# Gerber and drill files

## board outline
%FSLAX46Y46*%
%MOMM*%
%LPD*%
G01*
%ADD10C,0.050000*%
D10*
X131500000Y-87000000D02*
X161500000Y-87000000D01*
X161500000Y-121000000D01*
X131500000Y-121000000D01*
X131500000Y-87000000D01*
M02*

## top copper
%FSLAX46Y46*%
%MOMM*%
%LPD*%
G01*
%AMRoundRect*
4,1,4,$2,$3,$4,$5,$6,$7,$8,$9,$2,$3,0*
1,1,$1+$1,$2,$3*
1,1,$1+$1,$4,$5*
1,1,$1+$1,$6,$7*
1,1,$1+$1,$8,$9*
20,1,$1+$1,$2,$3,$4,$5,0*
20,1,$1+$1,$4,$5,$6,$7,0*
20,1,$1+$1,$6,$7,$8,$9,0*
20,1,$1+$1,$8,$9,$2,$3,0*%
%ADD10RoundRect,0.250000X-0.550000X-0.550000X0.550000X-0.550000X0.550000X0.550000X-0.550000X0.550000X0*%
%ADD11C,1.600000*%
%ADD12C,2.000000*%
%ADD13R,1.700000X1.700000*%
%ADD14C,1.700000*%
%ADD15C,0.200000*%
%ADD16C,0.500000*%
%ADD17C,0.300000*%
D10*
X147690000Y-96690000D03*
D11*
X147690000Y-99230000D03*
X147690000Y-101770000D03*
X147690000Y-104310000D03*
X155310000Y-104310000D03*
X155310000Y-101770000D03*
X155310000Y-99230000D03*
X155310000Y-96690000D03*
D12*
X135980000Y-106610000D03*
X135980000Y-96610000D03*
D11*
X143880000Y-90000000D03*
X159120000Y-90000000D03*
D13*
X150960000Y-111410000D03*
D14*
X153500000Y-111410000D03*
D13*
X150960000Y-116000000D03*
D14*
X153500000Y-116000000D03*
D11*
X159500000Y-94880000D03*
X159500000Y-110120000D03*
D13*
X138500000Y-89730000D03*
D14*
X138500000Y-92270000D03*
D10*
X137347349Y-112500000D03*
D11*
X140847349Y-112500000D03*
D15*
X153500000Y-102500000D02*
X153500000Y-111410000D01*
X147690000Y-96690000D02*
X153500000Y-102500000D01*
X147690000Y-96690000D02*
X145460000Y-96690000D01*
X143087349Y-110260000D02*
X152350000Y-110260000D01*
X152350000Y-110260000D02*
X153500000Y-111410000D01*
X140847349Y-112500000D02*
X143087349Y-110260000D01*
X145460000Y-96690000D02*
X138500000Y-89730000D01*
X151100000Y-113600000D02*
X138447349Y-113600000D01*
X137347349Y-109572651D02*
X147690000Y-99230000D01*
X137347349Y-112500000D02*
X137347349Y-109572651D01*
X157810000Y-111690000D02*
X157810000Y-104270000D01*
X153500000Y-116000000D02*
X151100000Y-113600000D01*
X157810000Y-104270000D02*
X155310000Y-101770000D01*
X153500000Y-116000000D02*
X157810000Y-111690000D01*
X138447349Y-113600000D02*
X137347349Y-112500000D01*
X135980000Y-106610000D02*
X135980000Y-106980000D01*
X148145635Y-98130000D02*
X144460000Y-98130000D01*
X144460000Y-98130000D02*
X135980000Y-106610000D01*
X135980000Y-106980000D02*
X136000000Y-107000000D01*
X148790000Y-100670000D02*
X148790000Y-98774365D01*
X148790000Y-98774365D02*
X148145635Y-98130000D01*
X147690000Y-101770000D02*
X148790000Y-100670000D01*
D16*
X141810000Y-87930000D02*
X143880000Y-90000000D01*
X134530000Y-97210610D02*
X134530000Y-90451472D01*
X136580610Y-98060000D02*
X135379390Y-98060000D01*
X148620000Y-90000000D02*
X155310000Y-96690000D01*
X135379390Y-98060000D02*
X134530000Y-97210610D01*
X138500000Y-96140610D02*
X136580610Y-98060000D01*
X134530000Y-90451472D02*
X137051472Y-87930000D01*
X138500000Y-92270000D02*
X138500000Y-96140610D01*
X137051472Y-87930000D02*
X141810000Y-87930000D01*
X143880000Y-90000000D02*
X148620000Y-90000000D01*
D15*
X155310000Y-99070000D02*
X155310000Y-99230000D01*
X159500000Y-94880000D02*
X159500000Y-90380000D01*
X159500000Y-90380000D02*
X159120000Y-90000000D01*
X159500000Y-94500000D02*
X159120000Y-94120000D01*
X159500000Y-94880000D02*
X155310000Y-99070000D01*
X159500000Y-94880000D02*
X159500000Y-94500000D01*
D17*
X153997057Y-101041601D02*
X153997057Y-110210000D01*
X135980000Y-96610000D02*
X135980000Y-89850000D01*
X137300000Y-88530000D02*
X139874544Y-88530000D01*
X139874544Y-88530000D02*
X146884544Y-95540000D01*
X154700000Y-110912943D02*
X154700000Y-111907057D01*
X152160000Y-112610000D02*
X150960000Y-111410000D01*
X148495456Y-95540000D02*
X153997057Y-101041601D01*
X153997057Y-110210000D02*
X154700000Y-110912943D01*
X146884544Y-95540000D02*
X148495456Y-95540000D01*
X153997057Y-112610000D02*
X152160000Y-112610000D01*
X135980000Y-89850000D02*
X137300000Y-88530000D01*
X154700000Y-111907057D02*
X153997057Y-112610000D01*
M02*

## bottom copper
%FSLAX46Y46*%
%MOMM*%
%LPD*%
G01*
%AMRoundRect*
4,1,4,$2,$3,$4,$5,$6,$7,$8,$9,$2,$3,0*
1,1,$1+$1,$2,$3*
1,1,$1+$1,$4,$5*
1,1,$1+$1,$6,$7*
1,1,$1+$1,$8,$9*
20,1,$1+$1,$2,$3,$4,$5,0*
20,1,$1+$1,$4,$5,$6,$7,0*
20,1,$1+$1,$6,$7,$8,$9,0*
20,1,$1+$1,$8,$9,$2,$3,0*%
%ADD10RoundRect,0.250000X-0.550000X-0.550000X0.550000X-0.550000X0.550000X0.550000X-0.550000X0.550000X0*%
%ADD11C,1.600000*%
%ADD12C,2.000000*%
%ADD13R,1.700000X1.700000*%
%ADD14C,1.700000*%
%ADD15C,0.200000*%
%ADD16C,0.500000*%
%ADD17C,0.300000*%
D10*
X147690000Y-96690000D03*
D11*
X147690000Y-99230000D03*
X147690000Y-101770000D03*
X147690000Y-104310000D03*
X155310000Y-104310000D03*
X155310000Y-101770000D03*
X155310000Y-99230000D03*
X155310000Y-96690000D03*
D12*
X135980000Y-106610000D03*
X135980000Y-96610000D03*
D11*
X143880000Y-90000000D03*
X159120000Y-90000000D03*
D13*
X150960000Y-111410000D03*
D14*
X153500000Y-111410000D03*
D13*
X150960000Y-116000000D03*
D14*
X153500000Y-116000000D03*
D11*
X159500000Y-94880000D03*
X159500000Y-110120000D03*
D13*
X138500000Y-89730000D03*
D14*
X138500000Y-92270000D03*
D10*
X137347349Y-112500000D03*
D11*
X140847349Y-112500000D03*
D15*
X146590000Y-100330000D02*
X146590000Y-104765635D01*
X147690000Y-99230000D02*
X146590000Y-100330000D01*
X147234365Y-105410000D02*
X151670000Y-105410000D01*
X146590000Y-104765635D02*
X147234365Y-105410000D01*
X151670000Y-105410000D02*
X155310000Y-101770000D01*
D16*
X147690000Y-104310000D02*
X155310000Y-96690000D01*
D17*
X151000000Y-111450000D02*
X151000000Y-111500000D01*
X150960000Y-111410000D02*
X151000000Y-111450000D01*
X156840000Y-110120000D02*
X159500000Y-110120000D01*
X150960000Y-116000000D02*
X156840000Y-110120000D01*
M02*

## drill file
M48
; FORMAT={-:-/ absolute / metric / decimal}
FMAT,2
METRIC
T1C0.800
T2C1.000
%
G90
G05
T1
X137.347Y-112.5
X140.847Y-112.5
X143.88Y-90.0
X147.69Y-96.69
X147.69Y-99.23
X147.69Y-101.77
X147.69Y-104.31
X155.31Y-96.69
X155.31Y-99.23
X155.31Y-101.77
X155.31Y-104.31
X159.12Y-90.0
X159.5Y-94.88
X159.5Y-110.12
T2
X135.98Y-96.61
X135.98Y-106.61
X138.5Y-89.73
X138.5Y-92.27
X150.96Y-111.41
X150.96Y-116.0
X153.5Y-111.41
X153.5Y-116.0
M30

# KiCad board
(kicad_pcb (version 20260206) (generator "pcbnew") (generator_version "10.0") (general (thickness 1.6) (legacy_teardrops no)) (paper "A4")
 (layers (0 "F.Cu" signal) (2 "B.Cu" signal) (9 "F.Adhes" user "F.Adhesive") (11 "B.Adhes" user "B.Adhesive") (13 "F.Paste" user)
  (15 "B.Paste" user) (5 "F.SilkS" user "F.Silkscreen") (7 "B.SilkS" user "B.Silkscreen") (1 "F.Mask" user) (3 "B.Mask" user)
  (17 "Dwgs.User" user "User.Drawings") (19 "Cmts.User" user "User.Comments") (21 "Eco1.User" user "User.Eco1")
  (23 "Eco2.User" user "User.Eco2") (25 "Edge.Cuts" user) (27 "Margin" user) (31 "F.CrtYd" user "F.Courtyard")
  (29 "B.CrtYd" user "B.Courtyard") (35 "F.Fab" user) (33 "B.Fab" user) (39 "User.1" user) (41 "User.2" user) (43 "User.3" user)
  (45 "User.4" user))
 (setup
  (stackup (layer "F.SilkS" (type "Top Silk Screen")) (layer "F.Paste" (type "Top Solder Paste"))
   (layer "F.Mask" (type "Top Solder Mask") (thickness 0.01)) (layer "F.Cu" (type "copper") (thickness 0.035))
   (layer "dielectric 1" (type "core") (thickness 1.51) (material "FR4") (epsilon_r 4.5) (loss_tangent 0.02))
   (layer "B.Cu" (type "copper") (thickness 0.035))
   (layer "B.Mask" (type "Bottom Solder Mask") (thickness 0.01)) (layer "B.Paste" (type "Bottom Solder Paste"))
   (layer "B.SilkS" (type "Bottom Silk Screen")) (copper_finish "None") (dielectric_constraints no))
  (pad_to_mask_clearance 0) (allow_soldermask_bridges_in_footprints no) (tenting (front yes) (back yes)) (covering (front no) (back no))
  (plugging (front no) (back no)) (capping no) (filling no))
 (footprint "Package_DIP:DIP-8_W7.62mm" (layer "F.Cu") (at 147.69 96.69)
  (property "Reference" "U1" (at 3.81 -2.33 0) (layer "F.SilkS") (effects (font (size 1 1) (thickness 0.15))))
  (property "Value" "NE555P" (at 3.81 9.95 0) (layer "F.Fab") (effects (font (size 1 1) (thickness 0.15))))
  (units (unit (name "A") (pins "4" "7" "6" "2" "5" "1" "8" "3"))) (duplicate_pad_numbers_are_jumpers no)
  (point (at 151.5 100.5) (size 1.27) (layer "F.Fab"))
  (pad "1" thru_hole roundrect (at 0 0) (size 1.6 1.6) (drill 0.8) (layers "*.Cu" "*.Mask") (remove_unused_layers no)
   (roundrect_rratio 0.15625) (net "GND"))
  (pad "2" thru_hole circle (at 0 2.54) (size 1.6 1.6) (drill 0.8) (layers "*.Cu" "*.Mask") (remove_unused_layers no) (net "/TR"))
  (pad "3" thru_hole circle (at 0 5.08) (size 1.6 1.6) (drill 0.8) (layers "*.Cu" "*.Mask") (remove_unused_layers no) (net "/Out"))
  (pad "4" thru_hole circle (at 0 7.62) (size 1.6 1.6) (drill 0.8) (layers "*.Cu" "*.Mask") (remove_unused_layers no) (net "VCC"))
  (pad "5" thru_hole circle (at 7.62 7.62) (size 1.6 1.6) (drill 0.8) (layers "*.Cu" "*.Mask") (remove_unused_layers no)
   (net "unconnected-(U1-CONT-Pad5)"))
  (pad "6" thru_hole circle (at 7.62 5.08) (size 1.6 1.6) (drill 0.8) (layers "*.Cu" "*.Mask") (remove_unused_layers no) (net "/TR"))
  (pad "7" thru_hole circle (at 7.62 2.54) (size 1.6 1.6) (drill 0.8) (layers "*.Cu" "*.Mask") (remove_unused_layers no) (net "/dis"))
  (pad "8" thru_hole circle (at 7.62 0) (size 1.6 1.6) (drill 0.8) (layers "*.Cu" "*.Mask") (remove_unused_layers no) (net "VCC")))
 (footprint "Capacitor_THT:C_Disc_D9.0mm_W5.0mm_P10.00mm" (layer "F.Cu") (at 135.98 106.61 90)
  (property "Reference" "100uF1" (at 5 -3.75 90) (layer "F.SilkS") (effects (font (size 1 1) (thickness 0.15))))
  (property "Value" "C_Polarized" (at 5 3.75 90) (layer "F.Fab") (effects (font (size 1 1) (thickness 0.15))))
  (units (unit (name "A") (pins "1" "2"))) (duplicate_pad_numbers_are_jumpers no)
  (pad "1" thru_hole circle (at 0 0 90) (size 2 2) (drill 1) (layers "*.Cu" "*.Mask") (remove_unused_layers no) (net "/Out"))
  (pad "2" thru_hole circle (at 10 0 90) (size 2 2) (drill 1) (layers "*.Cu" "*.Mask") (remove_unused_layers no) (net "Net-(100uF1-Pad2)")))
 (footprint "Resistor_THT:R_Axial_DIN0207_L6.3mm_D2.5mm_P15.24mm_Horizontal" (layer "F.Cu") (at 143.88 90)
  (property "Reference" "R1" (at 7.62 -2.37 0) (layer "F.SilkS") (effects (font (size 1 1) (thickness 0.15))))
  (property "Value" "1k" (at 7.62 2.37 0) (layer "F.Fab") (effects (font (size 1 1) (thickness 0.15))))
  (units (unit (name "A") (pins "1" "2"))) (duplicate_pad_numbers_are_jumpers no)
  (pad "1" thru_hole circle (at 0 0) (size 1.6 1.6) (drill 0.8) (layers "*.Cu" "*.Mask") (remove_unused_layers no) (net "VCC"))
  (pad "2" thru_hole circle (at 15.24 0) (size 1.6 1.6) (drill 0.8) (layers "*.Cu" "*.Mask") (remove_unused_layers no) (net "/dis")))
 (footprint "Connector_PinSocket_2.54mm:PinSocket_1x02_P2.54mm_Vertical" (layer "F.Cu") (at 150.96 111.41 90)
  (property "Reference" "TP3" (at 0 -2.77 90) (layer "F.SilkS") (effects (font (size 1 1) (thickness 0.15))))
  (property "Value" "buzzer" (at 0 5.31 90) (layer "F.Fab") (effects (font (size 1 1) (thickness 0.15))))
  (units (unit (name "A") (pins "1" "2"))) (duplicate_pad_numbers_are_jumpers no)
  (pad "1" thru_hole rect (at 0 0 90) (size 1.7 1.7) (drill 1) (layers "*.Cu" "*.Mask") (remove_unused_layers no) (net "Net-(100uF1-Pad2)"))
  (pad "2" thru_hole circle (at 0 2.54 90) (size 1.7 1.7) (drill 1) (layers "*.Cu" "*.Mask") (remove_unused_layers no) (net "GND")))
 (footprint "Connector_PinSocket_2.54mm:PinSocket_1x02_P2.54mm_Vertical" (layer "F.Cu") (at 150.96 116 90)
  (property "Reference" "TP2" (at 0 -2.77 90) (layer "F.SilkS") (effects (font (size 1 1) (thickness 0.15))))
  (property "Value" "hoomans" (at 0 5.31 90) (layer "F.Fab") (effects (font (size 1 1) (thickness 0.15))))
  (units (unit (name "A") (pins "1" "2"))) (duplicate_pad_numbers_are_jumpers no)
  (pad "1" thru_hole rect (at 0 0 90) (size 1.7 1.7) (drill 1) (layers "*.Cu" "*.Mask") (remove_unused_layers no) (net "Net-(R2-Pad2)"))
  (pad "2" thru_hole circle (at 0 2.54 90) (size 1.7 1.7) (drill 1) (layers "*.Cu" "*.Mask") (remove_unused_layers no) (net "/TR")))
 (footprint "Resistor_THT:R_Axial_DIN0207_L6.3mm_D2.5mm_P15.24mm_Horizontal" (layer "F.Cu") (at 159.5 94.88 -90)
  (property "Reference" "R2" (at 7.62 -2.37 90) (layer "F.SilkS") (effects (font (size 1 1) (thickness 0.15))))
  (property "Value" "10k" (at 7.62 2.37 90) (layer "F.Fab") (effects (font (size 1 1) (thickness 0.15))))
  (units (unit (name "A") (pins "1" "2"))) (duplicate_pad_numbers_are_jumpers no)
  (pad "1" thru_hole circle (at 0 0 270) (size 1.6 1.6) (drill 0.8) (layers "*.Cu" "*.Mask") (remove_unused_layers no) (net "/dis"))
  (pad "2" thru_hole circle (at 15.24 0 270) (size 1.6 1.6) (drill 0.8) (layers "*.Cu" "*.Mask") (remove_unused_layers no)
   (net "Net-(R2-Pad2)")))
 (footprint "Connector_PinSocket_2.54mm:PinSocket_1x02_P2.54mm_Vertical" (layer "F.Cu") (at 138.5 89.73)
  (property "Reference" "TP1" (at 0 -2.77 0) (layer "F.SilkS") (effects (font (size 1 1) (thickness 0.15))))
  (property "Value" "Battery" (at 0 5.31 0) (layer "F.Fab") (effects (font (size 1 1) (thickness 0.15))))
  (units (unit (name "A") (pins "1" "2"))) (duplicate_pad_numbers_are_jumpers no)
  (pad "1" thru_hole rect (at 0 0) (size 1.7 1.7) (drill 1) (layers "*.Cu" "*.Mask") (remove_unused_layers no) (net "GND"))
  (pad "2" thru_hole circle (at 0 2.54) (size 1.7 1.7) (drill 1) (layers "*.Cu" "*.Mask") (remove_unused_layers no) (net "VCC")))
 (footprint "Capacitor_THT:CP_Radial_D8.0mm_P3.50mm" (layer "F.Cu") (at 137.347349 112.5)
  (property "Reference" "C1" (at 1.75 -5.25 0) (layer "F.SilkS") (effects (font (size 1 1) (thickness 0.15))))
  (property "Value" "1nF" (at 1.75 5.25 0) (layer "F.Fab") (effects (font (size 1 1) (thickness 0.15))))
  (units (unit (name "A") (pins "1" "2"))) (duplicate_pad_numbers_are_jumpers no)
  (pad "1" thru_hole roundrect (at 0 0) (size 1.6 1.6) (drill 0.8) (layers "*.Cu" "*.Mask") (remove_unused_layers no)
   (roundrect_rratio 0.15625) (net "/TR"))
  (pad "2" thru_hole circle (at 3.5 0) (size 1.6 1.6) (drill 0.8) (layers "*.Cu" "*.Mask") (remove_unused_layers no) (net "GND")))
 (gr_rect (start 131.5 87) (end 161.5 121) (stroke (width 0.05) (type solid)) (fill no) (layer "Edge.Cuts"))
 (segment (start 153.5 102.5) (end 153.5 111.41) (width 0.2) (layer "F.Cu") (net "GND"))
 (segment (start 147.69 96.69) (end 153.5 102.5) (width 0.2) (layer "F.Cu") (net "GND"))
 (segment (start 147.69 96.69) (end 145.46 96.69) (width 0.2) (layer "F.Cu") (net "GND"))
 (segment (start 143.087349 110.26) (end 152.35 110.26) (width 0.2) (layer "F.Cu") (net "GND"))
 (segment (start 152.35 110.26) (end 153.5 111.41) (width 0.2) (layer "F.Cu") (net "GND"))
 (segment (start 140.847349 112.5) (end 143.087349 110.26) (width 0.2) (layer "F.Cu") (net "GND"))
 (segment (start 145.46 96.69) (end 138.5 89.73) (width 0.2) (layer "F.Cu") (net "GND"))
 (segment (start 151.1 113.6) (end 138.447349 113.6) (width 0.2) (layer "F.Cu") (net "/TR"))
 (segment (start 137.347349 109.572651) (end 147.69 99.23) (width 0.2) (layer "F.Cu") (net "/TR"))
 (segment (start 137.347349 112.5) (end 137.347349 109.572651) (width 0.2) (layer "F.Cu") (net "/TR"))
 (segment (start 157.81 111.69) (end 157.81 104.27) (width 0.2) (layer "F.Cu") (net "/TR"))
 (segment (start 153.5 116) (end 151.1 113.6) (width 0.2) (layer "F.Cu") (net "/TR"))
 (segment (start 157.81 104.27) (end 155.31 101.77) (width 0.2) (layer "F.Cu") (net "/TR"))
 (segment (start 153.5 116) (end 157.81 111.69) (width 0.2) (layer "F.Cu") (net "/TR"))
 (segment (start 138.447349 113.6) (end 137.347349 112.5) (width 0.2) (layer "F.Cu") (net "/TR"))
 (segment (start 146.59 100.33) (end 146.59 104.765635) (width 0.2) (layer "B.Cu") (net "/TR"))
 (segment (start 147.69 99.23) (end 146.59 100.33) (width 0.2) (layer "B.Cu") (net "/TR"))
 (segment (start 147.234365 105.41) (end 151.67 105.41) (width 0.2) (layer "B.Cu") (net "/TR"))
 (segment (start 146.59 104.765635) (end 147.234365 105.41) (width 0.2) (layer "B.Cu") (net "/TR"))
 (segment (start 151.67 105.41) (end 155.31 101.77) (width 0.2) (layer "B.Cu") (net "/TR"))
 (segment (start 135.98 106.61) (end 135.98 106.98) (width 0.2) (layer "F.Cu") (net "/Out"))
 (segment (start 148.145635 98.13) (end 144.46 98.13) (width 0.2) (layer "F.Cu") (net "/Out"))
 (segment (start 144.46 98.13) (end 135.98 106.61) (width 0.2) (layer "F.Cu") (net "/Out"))
 (segment (start 135.98 106.98) (end 136 107) (width 0.2) (layer "F.Cu") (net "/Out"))
 (segment (start 148.79 100.67) (end 148.79 98.774365) (width 0.2) (layer "F.Cu") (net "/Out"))
 (segment (start 148.79 98.774365) (end 148.145635 98.13) (width 0.2) (layer "F.Cu") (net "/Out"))
 (segment (start 147.69 101.77) (end 148.79 100.67) (width 0.2) (layer "F.Cu") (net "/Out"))
 (segment (start 141.81 87.93) (end 143.88 90) (width 0.5) (layer "F.Cu") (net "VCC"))
 (segment (start 134.53 97.21061) (end 134.53 90.451472) (width 0.5) (layer "F.Cu") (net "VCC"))
 (segment (start 136.58061 98.06) (end 135.37939 98.06) (width 0.5) (layer "F.Cu") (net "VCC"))
 (segment (start 148.62 90) (end 155.31 96.69) (width 0.5) (layer "F.Cu") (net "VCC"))
 (segment (start 135.37939 98.06) (end 134.53 97.21061) (width 0.5) (layer "F.Cu") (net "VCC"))
 (segment (start 138.5 96.14061) (end 136.58061 98.06) (width 0.5) (layer "F.Cu") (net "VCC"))
 (segment (start 134.53 90.451472) (end 137.051472 87.93) (width 0.5) (layer "F.Cu") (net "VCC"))
 (segment (start 138.5 92.27) (end 138.5 96.14061) (width 0.5) (layer "F.Cu") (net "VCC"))
 (segment (start 137.051472 87.93) (end 141.81 87.93) (width 0.5) (layer "F.Cu") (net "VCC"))
 (segment (start 143.88 90) (end 148.62 90) (width 0.5) (layer "F.Cu") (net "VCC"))
 (segment (start 147.69 104.31) (end 155.31 96.69) (width 0.5) (layer "B.Cu") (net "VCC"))
 (segment (start 155.31 99.07) (end 155.31 99.23) (width 0.2) (layer "F.Cu") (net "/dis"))
 (segment (start 159.5 94.88) (end 159.5 90.38) (width 0.2) (layer "F.Cu") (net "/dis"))
 (segment (start 159.5 90.38) (end 159.12 90) (width 0.2) (layer "F.Cu") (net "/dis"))
 (segment (start 159.5 94.5) (end 159.12 94.12) (width 0.2) (layer "F.Cu") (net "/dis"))
 (segment (start 159.5 94.88) (end 155.31 99.07) (width 0.2) (layer "F.Cu") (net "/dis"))
 (segment (start 159.5 94.88) (end 159.5 94.5) (width 0.2) (layer "F.Cu") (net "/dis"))
 (segment (start 153.997057 101.041601) (end 153.997057 110.21) (width 0.3) (layer "F.Cu") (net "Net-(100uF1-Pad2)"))
 (segment (start 135.98 96.61) (end 135.98 89.85) (width 0.3) (layer "F.Cu") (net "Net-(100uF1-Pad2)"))
 (segment (start 137.3 88.53) (end 139.874544 88.53) (width 0.3) (layer "F.Cu") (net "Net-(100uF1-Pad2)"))
 (segment (start 139.874544 88.53) (end 146.884544 95.54) (width 0.3) (layer "F.Cu") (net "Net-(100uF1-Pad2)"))
 (segment (start 154.7 110.912943) (end 154.7 111.907057) (width 0.3) (layer "F.Cu") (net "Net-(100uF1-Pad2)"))
 (segment (start 152.16 112.61) (end 150.96 111.41) (width 0.3) (layer "F.Cu") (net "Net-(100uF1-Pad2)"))
 (segment (start 148.495456 95.54) (end 153.997057 101.041601) (width 0.3) (layer "F.Cu") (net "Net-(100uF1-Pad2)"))
 (segment (start 153.997057 110.21) (end 154.7 110.912943) (width 0.3) (layer "F.Cu") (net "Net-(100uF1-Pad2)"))
 (segment (start 146.884544 95.54) (end 148.495456 95.54) (width 0.3) (layer "F.Cu") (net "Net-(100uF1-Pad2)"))
 (segment (start 153.997057 112.61) (end 152.16 112.61) (width 0.3) (layer "F.Cu") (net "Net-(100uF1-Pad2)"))
 (segment (start 135.98 89.85) (end 137.3 88.53) (width 0.3) (layer "F.Cu") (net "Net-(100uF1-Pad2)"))
 (segment (start 154.7 111.907057) (end 153.997057 112.61) (width 0.3) (layer "F.Cu") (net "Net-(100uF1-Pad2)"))
 (segment (start 151 111.45) (end 151 111.5) (width 0.3) (layer "B.Cu") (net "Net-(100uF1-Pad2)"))
 (segment (start 150.96 111.41) (end 151 111.45) (width 0.3) (layer "B.Cu") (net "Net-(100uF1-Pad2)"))
 (segment (start 156.84 110.12) (end 159.5 110.12) (width 0.3) (layer "B.Cu") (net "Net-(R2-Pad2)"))
 (segment (start 150.96 116) (end 156.84 110.12) (width 0.3) (layer "B.Cu") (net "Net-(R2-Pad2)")))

